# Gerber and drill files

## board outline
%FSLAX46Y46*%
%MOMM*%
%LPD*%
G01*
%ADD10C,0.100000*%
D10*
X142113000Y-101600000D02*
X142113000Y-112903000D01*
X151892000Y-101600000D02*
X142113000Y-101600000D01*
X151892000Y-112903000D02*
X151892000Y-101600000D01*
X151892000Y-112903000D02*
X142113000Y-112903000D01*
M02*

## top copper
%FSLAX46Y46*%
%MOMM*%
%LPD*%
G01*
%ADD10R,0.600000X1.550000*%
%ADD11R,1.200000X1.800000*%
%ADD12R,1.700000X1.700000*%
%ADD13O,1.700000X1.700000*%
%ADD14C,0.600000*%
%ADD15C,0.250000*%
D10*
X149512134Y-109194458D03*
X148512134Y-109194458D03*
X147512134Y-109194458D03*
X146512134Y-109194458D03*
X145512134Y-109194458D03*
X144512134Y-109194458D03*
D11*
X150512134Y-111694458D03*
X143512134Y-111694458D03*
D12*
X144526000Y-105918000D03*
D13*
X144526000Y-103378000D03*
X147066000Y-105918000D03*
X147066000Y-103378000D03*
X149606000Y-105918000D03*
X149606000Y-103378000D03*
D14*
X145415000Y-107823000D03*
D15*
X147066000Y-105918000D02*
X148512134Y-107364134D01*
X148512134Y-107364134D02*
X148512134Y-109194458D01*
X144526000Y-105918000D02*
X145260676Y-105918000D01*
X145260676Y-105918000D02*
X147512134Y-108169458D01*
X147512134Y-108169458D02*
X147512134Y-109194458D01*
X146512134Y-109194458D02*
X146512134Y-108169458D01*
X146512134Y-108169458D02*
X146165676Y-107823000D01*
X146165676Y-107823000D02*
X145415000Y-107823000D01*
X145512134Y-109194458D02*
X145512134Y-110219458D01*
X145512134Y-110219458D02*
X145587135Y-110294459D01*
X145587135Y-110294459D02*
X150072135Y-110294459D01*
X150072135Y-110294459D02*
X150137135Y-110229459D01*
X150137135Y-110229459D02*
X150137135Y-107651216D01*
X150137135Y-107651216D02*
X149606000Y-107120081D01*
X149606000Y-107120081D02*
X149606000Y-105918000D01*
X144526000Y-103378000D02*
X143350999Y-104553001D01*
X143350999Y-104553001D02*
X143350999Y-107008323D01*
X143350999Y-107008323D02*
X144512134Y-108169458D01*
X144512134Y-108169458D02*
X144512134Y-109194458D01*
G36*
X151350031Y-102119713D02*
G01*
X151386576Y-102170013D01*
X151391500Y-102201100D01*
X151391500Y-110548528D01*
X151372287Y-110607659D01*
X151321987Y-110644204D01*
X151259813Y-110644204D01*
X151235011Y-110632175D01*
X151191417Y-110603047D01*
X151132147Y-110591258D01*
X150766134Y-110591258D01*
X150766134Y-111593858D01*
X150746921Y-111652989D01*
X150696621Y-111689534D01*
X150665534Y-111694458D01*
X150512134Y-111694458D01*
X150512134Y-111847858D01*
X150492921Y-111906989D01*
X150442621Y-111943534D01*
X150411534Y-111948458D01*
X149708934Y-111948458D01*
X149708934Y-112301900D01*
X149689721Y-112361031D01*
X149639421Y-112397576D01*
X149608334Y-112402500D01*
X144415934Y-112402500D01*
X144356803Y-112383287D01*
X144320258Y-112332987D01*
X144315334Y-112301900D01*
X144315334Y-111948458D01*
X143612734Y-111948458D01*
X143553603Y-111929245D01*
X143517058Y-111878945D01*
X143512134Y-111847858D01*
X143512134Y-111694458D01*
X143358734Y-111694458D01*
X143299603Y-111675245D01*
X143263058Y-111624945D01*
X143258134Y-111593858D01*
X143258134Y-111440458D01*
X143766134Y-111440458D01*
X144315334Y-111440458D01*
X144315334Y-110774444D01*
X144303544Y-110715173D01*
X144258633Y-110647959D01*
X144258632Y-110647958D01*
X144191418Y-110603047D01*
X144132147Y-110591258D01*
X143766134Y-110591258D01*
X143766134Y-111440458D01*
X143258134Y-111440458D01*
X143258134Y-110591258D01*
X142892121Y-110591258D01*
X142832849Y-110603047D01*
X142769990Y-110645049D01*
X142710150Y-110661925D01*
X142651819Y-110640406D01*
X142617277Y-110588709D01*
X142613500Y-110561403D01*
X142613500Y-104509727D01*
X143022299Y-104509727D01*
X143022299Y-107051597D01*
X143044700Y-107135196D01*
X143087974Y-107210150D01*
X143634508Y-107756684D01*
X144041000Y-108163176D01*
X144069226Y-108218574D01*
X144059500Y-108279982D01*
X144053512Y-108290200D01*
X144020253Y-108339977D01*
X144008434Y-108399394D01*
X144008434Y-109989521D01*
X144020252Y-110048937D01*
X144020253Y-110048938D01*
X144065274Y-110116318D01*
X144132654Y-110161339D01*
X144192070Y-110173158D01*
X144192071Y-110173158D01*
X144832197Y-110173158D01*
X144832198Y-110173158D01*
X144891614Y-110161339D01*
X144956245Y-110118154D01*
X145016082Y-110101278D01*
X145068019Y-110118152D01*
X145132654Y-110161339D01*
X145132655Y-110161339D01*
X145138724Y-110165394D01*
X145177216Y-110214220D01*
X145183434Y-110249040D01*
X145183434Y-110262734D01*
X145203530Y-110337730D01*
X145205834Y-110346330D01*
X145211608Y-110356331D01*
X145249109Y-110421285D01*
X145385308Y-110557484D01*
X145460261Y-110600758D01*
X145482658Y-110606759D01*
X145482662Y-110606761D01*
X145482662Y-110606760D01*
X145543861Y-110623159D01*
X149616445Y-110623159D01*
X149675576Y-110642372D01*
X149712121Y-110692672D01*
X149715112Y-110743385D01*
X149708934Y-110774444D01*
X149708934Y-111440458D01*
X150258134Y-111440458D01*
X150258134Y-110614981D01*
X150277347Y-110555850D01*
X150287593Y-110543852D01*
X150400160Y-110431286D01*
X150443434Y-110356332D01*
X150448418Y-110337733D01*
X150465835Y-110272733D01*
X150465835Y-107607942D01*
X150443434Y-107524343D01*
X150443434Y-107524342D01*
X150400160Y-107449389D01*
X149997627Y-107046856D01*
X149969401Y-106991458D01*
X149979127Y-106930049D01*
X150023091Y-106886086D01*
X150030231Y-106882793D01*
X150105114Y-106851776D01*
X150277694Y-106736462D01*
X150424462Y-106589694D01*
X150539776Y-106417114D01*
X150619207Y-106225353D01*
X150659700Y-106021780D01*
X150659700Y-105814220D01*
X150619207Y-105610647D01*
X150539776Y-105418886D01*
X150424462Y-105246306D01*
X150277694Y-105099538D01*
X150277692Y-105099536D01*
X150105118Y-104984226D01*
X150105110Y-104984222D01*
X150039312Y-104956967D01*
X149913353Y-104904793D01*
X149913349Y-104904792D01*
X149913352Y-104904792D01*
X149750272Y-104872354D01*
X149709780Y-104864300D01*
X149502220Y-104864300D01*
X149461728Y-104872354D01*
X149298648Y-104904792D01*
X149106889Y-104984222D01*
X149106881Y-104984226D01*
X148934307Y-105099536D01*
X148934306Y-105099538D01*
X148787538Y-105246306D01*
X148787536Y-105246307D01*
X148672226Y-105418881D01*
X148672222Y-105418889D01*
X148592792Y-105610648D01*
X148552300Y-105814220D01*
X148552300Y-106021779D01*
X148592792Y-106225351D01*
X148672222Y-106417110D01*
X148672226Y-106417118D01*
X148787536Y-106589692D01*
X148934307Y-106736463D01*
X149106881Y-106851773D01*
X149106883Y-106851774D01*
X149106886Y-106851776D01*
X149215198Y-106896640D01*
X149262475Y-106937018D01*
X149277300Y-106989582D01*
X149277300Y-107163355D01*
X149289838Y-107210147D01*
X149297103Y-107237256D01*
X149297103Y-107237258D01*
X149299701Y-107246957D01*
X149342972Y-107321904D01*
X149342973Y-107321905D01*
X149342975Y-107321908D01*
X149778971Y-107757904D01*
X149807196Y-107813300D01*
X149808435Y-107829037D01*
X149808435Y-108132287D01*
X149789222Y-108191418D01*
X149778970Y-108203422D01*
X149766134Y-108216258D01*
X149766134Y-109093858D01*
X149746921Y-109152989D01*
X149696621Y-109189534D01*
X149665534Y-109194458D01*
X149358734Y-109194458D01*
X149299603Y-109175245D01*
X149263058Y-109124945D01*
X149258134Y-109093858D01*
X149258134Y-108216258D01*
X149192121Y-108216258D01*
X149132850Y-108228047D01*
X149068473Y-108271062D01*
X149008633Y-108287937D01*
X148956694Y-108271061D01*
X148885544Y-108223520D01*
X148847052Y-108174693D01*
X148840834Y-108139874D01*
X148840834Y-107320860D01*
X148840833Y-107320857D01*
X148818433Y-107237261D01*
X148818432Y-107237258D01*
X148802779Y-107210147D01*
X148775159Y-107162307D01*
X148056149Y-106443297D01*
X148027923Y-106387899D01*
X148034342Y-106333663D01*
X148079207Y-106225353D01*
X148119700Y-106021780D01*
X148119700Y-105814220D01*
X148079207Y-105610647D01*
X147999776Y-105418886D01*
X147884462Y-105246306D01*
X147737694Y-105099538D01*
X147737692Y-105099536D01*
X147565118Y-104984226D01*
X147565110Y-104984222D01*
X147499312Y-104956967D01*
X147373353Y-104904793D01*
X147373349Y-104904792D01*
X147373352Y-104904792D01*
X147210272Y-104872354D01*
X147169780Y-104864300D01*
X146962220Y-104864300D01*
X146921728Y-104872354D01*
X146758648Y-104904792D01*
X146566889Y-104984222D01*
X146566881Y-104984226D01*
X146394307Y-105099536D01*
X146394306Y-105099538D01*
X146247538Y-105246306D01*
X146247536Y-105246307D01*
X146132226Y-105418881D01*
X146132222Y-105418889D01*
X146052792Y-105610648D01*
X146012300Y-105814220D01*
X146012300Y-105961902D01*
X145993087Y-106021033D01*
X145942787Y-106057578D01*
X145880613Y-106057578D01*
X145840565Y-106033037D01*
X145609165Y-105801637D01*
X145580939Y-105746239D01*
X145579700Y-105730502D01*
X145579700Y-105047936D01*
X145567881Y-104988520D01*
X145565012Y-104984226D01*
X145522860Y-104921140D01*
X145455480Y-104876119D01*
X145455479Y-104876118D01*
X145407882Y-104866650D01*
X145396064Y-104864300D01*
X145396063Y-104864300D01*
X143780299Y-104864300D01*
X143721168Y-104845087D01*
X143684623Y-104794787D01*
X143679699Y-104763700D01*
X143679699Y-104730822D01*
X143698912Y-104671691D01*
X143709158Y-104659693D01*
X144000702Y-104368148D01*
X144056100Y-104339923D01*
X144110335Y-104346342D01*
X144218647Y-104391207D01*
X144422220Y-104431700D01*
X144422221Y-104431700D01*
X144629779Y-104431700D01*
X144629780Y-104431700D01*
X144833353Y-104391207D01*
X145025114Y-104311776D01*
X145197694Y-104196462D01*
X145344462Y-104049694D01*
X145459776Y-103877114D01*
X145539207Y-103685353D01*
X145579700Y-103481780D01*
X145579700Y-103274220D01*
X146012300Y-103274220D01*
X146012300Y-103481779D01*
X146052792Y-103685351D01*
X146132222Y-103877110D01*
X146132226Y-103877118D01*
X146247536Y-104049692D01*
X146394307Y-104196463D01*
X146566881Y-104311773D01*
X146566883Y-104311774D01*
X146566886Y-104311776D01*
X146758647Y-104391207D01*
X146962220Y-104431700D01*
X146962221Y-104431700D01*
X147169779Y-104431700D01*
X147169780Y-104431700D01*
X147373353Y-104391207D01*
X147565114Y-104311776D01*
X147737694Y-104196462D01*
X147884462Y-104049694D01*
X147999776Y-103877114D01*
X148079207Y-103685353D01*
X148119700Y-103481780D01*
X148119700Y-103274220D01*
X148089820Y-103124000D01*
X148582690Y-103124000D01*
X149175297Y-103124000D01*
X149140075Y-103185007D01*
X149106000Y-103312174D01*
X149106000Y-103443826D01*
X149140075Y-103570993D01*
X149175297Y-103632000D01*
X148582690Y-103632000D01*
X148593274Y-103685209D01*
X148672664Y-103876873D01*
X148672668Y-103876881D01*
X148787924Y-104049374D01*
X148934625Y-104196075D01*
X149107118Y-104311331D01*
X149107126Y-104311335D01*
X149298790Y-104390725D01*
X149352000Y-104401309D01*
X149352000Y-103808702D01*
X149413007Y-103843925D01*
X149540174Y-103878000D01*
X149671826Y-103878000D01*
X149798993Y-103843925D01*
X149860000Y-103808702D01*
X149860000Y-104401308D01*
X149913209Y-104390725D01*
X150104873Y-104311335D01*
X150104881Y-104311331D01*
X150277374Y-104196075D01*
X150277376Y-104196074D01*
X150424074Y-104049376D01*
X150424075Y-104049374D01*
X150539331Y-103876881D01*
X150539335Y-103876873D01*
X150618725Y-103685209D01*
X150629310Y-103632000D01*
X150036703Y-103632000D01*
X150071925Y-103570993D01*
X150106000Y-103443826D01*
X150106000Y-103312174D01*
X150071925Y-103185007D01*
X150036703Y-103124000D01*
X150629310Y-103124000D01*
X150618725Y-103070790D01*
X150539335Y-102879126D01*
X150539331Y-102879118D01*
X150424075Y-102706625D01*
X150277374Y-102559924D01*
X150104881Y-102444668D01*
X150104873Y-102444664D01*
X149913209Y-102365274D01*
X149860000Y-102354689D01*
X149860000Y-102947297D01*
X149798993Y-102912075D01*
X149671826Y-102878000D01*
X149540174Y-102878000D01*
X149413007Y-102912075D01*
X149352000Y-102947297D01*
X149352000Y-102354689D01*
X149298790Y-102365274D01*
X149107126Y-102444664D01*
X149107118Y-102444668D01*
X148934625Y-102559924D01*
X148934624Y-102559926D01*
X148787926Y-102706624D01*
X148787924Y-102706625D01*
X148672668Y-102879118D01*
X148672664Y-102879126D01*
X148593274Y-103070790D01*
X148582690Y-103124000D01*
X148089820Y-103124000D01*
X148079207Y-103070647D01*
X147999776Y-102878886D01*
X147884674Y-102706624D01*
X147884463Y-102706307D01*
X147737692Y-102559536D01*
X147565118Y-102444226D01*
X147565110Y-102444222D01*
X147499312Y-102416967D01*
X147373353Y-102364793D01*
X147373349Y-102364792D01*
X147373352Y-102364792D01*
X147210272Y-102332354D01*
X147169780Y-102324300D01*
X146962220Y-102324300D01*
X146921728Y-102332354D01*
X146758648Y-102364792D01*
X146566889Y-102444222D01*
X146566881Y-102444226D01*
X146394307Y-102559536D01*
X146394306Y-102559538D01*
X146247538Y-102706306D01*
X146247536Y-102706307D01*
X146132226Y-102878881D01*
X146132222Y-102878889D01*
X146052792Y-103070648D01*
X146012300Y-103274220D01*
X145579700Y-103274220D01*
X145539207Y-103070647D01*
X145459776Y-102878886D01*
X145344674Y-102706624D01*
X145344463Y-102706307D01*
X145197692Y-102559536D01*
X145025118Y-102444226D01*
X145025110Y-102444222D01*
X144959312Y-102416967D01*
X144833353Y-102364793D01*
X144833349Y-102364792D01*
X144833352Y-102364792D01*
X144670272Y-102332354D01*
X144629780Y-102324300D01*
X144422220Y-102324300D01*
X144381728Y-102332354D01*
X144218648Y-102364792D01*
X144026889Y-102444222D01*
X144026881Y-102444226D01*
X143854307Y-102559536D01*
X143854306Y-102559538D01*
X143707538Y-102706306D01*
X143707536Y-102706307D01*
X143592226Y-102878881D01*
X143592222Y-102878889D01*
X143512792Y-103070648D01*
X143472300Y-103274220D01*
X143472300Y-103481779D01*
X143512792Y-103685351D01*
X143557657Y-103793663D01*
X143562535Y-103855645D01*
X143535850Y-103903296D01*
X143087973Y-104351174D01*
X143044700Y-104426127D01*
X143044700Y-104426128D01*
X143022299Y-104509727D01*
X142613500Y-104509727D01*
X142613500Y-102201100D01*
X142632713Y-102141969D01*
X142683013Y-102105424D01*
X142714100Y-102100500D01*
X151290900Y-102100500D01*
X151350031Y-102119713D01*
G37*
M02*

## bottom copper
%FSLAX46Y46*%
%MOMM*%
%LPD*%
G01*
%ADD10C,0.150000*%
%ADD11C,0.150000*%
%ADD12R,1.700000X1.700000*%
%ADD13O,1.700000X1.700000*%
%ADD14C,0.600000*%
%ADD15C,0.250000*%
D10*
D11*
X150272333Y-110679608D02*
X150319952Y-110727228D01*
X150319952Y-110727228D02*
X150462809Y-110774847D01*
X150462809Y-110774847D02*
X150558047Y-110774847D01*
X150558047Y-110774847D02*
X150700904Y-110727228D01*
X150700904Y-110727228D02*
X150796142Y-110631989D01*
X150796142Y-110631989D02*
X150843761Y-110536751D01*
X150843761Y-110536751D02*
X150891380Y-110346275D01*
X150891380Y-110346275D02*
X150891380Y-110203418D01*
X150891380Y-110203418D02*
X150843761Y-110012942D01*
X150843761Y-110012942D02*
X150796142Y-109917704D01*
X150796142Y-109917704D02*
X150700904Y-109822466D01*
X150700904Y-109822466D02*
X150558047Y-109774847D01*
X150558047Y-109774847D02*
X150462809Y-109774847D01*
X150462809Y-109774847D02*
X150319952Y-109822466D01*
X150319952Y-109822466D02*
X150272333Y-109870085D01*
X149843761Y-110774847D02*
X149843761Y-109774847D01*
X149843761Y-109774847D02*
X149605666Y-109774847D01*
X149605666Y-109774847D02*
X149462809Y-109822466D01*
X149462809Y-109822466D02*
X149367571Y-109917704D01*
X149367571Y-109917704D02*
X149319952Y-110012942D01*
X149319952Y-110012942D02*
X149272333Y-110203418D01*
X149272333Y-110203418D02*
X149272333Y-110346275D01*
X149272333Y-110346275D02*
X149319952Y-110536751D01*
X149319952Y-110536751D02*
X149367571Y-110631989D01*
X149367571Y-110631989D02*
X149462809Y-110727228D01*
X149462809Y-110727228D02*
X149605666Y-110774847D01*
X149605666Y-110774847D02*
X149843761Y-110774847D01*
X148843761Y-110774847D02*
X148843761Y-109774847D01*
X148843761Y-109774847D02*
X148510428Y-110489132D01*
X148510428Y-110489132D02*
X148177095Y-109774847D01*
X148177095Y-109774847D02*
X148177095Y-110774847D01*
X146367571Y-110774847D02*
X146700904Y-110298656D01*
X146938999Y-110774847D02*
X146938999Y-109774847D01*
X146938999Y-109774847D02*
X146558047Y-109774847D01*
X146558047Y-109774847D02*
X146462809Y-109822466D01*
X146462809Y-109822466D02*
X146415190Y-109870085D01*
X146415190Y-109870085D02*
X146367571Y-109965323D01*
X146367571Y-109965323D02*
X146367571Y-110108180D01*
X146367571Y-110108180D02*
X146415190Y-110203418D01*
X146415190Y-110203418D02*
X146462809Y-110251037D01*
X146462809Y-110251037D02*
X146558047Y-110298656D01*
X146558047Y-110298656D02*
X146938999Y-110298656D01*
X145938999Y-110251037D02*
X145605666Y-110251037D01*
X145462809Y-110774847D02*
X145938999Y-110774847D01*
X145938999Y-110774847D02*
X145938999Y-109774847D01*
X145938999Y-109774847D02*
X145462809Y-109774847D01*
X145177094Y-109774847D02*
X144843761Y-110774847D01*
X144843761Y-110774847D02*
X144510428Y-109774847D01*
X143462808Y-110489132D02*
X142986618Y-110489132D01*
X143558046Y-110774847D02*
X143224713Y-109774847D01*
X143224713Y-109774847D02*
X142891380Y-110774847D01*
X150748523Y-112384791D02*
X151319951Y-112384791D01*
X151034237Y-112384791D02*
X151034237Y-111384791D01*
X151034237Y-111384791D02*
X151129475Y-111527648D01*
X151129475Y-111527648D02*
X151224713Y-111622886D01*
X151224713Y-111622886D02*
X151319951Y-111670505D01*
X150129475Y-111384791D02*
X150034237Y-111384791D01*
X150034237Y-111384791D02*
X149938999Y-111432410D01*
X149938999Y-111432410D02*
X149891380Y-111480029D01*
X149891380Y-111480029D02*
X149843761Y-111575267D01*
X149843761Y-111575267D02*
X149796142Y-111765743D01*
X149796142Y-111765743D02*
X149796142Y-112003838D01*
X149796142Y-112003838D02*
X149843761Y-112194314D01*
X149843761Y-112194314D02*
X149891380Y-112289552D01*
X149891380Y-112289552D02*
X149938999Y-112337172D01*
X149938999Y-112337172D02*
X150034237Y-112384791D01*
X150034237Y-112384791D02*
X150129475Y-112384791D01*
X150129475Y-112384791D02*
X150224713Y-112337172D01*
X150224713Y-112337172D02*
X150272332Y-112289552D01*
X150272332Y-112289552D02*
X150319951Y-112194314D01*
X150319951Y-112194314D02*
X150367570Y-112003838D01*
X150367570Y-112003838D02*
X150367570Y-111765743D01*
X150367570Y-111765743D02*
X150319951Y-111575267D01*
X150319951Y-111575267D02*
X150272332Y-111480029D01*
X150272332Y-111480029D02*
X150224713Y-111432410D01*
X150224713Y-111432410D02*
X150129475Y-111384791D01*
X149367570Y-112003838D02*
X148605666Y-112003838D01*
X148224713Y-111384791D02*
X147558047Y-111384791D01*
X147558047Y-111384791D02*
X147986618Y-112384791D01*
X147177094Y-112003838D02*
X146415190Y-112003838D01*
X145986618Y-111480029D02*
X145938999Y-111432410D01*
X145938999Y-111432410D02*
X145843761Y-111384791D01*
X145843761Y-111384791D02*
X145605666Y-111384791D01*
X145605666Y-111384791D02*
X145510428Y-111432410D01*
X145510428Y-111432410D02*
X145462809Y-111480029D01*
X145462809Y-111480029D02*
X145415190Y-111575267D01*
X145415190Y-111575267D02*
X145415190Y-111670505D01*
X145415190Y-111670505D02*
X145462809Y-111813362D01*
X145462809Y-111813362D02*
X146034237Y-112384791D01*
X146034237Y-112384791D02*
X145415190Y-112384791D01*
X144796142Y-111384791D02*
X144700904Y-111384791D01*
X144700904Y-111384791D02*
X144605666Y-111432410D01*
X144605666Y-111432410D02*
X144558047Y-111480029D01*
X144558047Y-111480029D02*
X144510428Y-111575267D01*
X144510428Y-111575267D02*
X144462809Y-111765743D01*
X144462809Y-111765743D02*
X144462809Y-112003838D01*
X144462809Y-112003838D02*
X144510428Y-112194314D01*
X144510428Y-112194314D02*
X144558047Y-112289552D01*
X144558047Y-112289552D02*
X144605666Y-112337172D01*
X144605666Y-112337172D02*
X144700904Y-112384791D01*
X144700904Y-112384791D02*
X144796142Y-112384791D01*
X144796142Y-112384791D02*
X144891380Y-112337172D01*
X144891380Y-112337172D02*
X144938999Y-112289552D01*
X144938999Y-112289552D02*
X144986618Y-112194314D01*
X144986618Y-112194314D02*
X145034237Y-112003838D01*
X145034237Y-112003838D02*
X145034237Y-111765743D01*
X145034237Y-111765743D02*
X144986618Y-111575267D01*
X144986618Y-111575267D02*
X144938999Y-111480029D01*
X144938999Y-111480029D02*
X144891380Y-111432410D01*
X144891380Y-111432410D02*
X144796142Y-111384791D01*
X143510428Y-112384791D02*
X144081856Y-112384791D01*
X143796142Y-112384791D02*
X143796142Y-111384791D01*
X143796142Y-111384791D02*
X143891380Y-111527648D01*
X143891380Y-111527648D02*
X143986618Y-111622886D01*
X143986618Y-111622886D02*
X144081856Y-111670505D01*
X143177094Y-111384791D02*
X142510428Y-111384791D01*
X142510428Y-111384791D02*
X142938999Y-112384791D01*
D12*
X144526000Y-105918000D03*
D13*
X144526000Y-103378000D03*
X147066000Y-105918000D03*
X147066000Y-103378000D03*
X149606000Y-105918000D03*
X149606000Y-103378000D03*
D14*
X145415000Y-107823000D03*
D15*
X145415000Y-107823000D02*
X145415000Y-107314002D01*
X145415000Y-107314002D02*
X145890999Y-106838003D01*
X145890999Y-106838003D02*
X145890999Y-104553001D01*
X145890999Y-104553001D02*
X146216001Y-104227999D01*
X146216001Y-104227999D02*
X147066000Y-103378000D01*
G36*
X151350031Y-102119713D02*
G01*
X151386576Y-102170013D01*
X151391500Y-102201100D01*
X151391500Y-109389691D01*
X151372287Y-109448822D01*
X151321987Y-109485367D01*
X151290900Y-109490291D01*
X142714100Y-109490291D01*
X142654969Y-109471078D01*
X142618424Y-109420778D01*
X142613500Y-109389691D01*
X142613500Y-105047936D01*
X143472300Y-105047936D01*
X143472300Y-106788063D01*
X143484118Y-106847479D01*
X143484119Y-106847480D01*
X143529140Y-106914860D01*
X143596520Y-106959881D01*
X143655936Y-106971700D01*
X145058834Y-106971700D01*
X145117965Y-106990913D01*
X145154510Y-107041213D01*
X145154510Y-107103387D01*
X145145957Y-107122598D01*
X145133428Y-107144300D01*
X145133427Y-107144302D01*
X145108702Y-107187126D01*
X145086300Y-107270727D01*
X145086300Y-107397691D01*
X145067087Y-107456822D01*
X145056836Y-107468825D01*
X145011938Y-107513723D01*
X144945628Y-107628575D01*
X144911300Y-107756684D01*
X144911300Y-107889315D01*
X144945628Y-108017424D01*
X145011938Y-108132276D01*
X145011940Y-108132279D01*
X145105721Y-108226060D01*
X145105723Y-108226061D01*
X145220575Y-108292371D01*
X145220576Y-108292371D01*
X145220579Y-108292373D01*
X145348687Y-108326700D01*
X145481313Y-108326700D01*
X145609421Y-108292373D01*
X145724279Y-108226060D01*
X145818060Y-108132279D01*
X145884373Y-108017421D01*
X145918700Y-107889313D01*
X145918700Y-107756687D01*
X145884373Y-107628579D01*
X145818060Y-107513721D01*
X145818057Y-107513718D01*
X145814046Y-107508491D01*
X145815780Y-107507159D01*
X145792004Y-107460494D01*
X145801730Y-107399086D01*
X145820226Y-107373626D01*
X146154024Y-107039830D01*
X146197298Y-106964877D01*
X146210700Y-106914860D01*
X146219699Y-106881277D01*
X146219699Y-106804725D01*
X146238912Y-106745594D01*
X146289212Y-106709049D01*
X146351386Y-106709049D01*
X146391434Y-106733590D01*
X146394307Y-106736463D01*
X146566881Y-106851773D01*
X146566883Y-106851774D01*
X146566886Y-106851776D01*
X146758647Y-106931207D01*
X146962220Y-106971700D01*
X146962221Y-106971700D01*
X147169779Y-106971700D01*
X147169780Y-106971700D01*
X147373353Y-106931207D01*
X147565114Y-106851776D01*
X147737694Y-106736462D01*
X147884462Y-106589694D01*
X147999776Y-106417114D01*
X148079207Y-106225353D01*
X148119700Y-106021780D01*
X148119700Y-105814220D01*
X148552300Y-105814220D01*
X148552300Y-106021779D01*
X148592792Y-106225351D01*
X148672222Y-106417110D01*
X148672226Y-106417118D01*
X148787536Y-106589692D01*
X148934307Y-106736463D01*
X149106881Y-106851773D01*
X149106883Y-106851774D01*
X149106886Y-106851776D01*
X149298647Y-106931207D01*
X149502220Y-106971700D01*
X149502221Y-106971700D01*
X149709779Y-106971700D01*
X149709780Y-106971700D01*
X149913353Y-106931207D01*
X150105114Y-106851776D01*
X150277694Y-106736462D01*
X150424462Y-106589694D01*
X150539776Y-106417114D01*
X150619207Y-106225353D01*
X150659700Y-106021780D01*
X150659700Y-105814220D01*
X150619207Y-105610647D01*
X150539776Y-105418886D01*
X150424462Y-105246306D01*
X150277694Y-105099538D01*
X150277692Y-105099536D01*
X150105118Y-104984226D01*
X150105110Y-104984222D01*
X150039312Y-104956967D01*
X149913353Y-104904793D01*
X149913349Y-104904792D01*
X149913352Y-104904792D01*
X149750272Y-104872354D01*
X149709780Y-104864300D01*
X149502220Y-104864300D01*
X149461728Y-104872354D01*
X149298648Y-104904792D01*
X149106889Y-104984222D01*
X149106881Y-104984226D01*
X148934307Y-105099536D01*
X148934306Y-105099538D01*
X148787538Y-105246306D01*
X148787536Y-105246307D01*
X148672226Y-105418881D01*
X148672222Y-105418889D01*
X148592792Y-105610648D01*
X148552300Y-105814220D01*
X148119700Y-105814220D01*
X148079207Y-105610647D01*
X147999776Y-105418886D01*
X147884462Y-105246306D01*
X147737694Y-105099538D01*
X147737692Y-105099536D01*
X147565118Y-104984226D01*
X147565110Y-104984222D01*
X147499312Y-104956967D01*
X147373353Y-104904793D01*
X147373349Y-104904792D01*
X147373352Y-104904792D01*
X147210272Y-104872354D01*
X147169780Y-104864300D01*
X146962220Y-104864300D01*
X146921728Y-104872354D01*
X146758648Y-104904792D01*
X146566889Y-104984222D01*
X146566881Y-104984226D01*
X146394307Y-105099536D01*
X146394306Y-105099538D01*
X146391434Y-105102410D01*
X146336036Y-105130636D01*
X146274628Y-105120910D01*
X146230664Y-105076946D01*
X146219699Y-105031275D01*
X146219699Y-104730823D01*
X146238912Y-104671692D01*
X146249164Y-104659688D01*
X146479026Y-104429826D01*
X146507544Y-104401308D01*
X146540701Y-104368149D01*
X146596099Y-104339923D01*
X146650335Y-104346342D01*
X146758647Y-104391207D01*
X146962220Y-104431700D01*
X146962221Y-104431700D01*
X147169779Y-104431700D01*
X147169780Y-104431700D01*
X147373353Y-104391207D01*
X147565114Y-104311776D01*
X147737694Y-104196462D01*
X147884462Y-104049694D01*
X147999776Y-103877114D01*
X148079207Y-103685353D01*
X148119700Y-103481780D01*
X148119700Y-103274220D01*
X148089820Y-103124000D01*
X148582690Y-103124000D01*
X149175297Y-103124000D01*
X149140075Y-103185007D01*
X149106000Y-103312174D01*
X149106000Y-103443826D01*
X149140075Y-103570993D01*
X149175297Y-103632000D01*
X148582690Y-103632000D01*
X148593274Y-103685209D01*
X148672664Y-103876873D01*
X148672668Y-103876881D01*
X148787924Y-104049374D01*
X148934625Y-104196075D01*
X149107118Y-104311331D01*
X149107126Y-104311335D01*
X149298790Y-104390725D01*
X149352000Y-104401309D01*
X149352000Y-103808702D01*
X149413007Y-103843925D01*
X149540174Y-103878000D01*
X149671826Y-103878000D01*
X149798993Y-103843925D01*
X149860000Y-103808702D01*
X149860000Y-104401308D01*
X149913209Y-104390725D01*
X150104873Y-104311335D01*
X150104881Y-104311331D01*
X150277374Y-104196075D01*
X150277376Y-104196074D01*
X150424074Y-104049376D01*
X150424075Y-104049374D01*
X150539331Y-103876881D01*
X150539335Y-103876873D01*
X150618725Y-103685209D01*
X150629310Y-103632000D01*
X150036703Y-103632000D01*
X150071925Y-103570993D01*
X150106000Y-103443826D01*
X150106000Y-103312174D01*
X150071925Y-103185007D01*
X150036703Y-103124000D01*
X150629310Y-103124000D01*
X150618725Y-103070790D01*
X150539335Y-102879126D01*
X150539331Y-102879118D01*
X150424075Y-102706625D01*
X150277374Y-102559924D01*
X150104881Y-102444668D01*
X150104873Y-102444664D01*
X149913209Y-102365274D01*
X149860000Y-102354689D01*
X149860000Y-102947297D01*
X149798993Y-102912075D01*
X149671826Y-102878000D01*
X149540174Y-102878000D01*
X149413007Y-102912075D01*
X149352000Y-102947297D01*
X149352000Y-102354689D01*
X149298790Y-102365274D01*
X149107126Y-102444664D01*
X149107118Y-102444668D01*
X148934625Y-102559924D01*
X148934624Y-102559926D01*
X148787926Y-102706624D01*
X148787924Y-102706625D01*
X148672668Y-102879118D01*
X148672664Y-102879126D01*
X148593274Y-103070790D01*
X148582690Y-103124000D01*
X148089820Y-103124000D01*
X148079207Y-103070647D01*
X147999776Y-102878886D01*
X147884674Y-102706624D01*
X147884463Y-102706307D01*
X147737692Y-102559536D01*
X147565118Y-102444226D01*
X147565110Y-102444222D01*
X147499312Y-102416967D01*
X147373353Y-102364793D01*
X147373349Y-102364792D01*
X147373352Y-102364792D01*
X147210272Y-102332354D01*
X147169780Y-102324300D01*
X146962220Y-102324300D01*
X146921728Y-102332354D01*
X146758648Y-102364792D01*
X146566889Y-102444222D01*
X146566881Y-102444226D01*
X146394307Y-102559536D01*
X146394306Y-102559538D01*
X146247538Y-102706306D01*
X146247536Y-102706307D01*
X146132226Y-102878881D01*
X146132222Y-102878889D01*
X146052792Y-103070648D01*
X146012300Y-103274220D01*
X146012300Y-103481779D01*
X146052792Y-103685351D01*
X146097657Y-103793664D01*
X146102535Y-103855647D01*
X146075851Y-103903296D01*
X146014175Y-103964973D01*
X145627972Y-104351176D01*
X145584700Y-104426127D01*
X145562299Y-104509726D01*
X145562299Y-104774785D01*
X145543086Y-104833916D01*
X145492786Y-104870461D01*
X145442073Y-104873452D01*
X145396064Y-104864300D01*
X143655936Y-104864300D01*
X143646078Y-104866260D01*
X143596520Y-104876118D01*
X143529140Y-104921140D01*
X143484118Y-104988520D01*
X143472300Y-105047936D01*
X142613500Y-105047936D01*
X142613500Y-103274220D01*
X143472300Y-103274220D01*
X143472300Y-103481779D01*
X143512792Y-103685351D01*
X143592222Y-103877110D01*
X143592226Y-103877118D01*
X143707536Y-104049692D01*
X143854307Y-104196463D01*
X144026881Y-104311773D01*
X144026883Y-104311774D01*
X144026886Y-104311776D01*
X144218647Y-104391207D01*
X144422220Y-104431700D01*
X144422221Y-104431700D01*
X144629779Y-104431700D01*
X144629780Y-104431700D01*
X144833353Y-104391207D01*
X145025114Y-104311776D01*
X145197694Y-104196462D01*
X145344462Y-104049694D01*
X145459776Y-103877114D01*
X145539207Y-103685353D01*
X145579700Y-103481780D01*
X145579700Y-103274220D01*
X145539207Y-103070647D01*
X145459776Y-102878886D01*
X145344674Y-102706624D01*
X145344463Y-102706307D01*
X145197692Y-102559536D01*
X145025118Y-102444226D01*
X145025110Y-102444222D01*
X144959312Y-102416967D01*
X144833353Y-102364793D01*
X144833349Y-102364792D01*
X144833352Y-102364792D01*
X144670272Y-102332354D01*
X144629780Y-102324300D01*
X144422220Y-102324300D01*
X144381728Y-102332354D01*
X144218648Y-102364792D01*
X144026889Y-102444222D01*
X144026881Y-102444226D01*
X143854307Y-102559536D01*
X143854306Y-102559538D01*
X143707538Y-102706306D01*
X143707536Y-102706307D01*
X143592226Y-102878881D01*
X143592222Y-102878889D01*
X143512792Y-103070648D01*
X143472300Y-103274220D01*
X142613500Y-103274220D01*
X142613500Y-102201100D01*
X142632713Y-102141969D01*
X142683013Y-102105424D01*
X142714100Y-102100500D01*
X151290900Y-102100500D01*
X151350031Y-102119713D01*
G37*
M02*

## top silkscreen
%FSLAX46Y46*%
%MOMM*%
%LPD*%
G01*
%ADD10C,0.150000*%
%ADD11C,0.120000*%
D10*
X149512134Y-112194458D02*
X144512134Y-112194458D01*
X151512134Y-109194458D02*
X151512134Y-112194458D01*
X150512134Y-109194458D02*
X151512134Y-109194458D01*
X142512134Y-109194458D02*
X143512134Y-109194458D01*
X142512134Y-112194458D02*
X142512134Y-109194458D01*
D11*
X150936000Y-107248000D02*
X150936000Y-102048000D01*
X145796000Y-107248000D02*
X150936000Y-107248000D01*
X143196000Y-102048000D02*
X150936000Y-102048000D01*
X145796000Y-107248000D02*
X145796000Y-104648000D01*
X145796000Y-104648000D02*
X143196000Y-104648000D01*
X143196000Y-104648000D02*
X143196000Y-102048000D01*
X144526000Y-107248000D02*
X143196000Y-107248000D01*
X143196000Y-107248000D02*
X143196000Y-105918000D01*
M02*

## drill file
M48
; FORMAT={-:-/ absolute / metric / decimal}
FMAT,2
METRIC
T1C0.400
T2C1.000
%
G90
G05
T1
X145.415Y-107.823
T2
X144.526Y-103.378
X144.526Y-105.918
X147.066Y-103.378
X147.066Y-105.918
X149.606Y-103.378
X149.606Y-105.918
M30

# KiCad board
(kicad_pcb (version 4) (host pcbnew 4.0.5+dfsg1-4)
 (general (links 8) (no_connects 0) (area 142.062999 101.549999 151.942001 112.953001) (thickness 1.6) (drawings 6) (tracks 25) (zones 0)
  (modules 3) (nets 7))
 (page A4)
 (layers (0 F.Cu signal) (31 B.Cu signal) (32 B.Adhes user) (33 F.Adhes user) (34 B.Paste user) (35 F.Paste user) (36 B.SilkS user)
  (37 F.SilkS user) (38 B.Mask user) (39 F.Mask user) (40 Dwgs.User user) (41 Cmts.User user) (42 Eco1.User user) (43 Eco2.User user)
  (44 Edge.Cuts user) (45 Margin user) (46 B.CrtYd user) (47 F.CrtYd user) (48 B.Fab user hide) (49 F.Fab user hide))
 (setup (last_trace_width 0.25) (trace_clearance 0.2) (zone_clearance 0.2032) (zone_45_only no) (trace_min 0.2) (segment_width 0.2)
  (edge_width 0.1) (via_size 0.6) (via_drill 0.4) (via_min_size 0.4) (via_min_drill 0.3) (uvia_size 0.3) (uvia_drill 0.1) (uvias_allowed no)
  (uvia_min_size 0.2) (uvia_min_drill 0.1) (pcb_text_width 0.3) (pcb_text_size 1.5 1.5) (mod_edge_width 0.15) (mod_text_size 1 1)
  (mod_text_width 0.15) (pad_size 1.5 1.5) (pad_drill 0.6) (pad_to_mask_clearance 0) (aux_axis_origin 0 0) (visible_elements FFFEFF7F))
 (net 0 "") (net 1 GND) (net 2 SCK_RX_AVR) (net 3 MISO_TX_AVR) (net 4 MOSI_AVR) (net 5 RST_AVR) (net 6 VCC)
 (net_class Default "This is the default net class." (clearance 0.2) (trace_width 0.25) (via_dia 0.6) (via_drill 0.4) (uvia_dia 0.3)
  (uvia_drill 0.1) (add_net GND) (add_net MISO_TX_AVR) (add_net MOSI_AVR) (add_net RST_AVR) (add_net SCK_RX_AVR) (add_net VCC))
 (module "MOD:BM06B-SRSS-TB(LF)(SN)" (layer F.Cu) (at 148.5011 105.0036)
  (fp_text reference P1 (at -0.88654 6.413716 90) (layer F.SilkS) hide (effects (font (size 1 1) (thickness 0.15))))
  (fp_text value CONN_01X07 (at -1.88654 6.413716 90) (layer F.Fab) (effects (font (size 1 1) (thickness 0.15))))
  (fp_line (start 1.011034 7.190858) (end -3.988966 7.190858) (layer F.SilkS) (width 0.15))
  (fp_line (start 3.011034 4.190858) (end 3.011034 7.190858) (layer F.SilkS) (width 0.15))
  (fp_line (start 2.011034 4.190858) (end 3.011034 4.190858) (layer F.SilkS) (width 0.15))
  (fp_line (start -5.988966 4.190858) (end -4.988966 4.190858) (layer F.SilkS) (width 0.15))
  (fp_line (start -5.988966 7.190858) (end -5.988966 4.190858) (layer F.SilkS) (width 0.15))
  (pad 6 smd rect (at 1.011034 4.190858 180) (size 0.6 1.55) (layers F.Cu F.Paste F.Mask) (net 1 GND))
  (pad 5 smd rect (at 0.011034 4.190858 180) (size 0.6 1.55) (layers F.Cu F.Paste F.Mask) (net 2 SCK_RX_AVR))
  (pad 4 smd rect (at -0.988966 4.190858 180) (size 0.6 1.55) (layers F.Cu F.Paste F.Mask) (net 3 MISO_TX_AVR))
  (pad 3 smd rect (at -1.988966 4.190858 180) (size 0.6 1.55) (layers F.Cu F.Paste F.Mask) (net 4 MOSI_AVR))
  (pad 2 smd rect (at -2.988966 4.190858 180) (size 0.6 1.55) (layers F.Cu F.Paste F.Mask) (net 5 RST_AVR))
  (pad 1 smd rect (at -3.988966 4.190858 180) (size 0.6 1.55) (layers F.Cu F.Paste F.Mask) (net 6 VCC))
  (pad 7 smd rect (at 2.011034 6.690858 180) (size 1.2 1.8) (layers F.Cu F.Paste F.Mask) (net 1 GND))
  (pad 7 smd rect (at -4.988966 6.690858 180) (size 1.2 1.8) (layers F.Cu F.Paste F.Mask) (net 1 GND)))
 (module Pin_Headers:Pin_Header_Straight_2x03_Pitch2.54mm (layer F.Cu) (at 144.526 105.918 90)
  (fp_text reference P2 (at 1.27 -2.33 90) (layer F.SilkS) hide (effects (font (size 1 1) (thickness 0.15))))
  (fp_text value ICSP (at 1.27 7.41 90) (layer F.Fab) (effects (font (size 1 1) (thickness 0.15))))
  (fp_line (start -1.33 6.41) (end 3.87 6.41) (layer F.SilkS) (width 0.12))
  (fp_line (start -1.33 1.27) (end -1.33 6.41) (layer F.SilkS) (width 0.12))
  (fp_line (start 3.87 -1.33) (end 3.87 6.41) (layer F.SilkS) (width 0.12))
  (fp_line (start -1.33 1.27) (end 1.27 1.27) (layer F.SilkS) (width 0.12))
  (fp_line (start 1.27 1.27) (end 1.27 -1.33) (layer F.SilkS) (width 0.12))
  (fp_line (start 1.27 -1.33) (end 3.87 -1.33) (layer F.SilkS) (width 0.12))
  (fp_line (start -1.33 0) (end -1.33 -1.33) (layer F.SilkS) (width 0.12))
  (fp_line (start -1.33 -1.33) (end 0 -1.33) (layer F.SilkS) (width 0.12))
  (pad 1 thru_hole rect (at 0 0 90) (size 1.7 1.7) (drill 1) (layers *.Cu *.Mask) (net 3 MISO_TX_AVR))
  (pad 2 thru_hole oval (at 2.54 0 90) (size 1.7 1.7) (drill 1) (layers *.Cu *.Mask) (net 6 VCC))
  (pad 3 thru_hole oval (at 0 2.54 90) (size 1.7 1.7) (drill 1) (layers *.Cu *.Mask) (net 2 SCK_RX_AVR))
  (pad 4 thru_hole oval (at 2.54 2.54 90) (size 1.7 1.7) (drill 1) (layers *.Cu *.Mask) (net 4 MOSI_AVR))
  (pad 5 thru_hole oval (at 0 5.08 90) (size 1.7 1.7) (drill 1) (layers *.Cu *.Mask) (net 5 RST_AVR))
  (pad 6 thru_hole oval (at 2.54 5.08 90) (size 1.7 1.7) (drill 1) (layers *.Cu *.Mask) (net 1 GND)))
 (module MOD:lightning (layer B.Cu) (at 149.86 111.125)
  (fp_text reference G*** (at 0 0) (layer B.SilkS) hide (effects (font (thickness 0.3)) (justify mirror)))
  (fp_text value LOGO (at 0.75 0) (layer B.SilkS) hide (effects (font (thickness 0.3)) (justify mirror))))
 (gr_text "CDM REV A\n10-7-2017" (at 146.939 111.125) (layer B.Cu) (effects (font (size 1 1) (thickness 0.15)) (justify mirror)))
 (gr_line (start 142.113 101.6) (end 142.113 112.903) (layer Edge.Cuts) (width 0.1))
 (gr_line (start 151.892 101.6) (end 142.113 101.6) (layer Edge.Cuts) (width 0.1))
 (gr_line (start 151.892 112.903) (end 151.892 101.6) (layer Edge.Cuts) (width 0.1))
 (gr_line (start 151.892 112.903) (end 142.113 112.903) (layer Edge.Cuts) (width 0.1))
 (segment (start 147.066 105.918) (end 148.512134 107.364134) (width 0.25) (layer F.Cu) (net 2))
 (segment (start 148.512134 107.364134) (end 148.512134 109.194458) (width 0.25) (layer F.Cu) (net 2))
 (segment (start 144.526 105.918) (end 145.260676 105.918) (width 0.25) (layer F.Cu) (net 3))
 (segment (start 145.260676 105.918) (end 147.512134 108.169458) (width 0.25) (layer F.Cu) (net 3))
 (segment (start 147.512134 108.169458) (end 147.512134 109.194458) (width 0.25) (layer F.Cu) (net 3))
 (segment (start 145.415 107.823) (end 145.415 107.314002) (width 0.25) (layer B.Cu) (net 4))
 (segment (start 145.415 107.314002) (end 145.890999 106.838003) (width 0.25) (layer B.Cu) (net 4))
 (segment (start 145.890999 106.838003) (end 145.890999 104.553001) (width 0.25) (layer B.Cu) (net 4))
 (segment (start 145.890999 104.553001) (end 146.216001 104.227999) (width 0.25) (layer B.Cu) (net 4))
 (segment (start 146.216001 104.227999) (end 147.066 103.378) (width 0.25) (layer B.Cu) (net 4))
 (segment (start 146.512134 109.194458) (end 146.512134 108.169458) (width 0.25) (layer F.Cu) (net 4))
 (via (at 145.415 107.823) (size 0.6) (drill 0.4) (layers F.Cu B.Cu) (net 4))
 (segment (start 146.512134 108.169458) (end 146.165676 107.823) (width 0.25) (layer F.Cu) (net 4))
 (segment (start 146.165676 107.823) (end 145.415 107.823) (width 0.25) (layer F.Cu) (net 4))
 (segment (start 145.512134 109.194458) (end 145.512134 110.219458) (width 0.25) (layer F.Cu) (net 5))
 (segment (start 145.512134 110.219458) (end 145.587135 110.294459) (width 0.25) (layer F.Cu) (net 5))
 (segment (start 145.587135 110.294459) (end 150.072135 110.294459) (width 0.25) (layer F.Cu) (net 5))
 (segment (start 150.072135 110.294459) (end 150.137135 110.229459) (width 0.25) (layer F.Cu) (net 5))
 (segment (start 150.137135 110.229459) (end 150.137135 107.651216) (width 0.25) (layer F.Cu) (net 5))
 (segment (start 150.137135 107.651216) (end 149.606 107.120081) (width 0.25) (layer F.Cu) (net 5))
 (segment (start 149.606 107.120081) (end 149.606 105.918) (width 0.25) (layer F.Cu) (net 5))
 (segment (start 144.526 103.378) (end 143.350999 104.553001) (width 0.25) (layer F.Cu) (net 6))
 (segment (start 143.350999 104.553001) (end 143.350999 107.008323) (width 0.25) (layer F.Cu) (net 6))
 (segment (start 143.350999 107.008323) (end 144.512134 108.169458) (width 0.25) (layer F.Cu) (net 6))
 (segment (start 144.512134 108.169458) (end 144.512134 109.194458) (width 0.25) (layer F.Cu) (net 6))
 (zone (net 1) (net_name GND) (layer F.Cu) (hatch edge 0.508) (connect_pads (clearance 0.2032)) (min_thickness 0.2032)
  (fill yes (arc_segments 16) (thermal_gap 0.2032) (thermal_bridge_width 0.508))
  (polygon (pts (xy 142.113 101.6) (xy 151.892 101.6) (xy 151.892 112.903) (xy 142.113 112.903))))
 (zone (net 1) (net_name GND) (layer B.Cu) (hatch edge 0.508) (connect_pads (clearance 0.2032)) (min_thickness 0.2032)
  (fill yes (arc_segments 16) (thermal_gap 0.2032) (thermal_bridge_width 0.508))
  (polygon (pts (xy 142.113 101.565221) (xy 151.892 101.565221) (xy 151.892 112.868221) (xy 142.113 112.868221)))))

